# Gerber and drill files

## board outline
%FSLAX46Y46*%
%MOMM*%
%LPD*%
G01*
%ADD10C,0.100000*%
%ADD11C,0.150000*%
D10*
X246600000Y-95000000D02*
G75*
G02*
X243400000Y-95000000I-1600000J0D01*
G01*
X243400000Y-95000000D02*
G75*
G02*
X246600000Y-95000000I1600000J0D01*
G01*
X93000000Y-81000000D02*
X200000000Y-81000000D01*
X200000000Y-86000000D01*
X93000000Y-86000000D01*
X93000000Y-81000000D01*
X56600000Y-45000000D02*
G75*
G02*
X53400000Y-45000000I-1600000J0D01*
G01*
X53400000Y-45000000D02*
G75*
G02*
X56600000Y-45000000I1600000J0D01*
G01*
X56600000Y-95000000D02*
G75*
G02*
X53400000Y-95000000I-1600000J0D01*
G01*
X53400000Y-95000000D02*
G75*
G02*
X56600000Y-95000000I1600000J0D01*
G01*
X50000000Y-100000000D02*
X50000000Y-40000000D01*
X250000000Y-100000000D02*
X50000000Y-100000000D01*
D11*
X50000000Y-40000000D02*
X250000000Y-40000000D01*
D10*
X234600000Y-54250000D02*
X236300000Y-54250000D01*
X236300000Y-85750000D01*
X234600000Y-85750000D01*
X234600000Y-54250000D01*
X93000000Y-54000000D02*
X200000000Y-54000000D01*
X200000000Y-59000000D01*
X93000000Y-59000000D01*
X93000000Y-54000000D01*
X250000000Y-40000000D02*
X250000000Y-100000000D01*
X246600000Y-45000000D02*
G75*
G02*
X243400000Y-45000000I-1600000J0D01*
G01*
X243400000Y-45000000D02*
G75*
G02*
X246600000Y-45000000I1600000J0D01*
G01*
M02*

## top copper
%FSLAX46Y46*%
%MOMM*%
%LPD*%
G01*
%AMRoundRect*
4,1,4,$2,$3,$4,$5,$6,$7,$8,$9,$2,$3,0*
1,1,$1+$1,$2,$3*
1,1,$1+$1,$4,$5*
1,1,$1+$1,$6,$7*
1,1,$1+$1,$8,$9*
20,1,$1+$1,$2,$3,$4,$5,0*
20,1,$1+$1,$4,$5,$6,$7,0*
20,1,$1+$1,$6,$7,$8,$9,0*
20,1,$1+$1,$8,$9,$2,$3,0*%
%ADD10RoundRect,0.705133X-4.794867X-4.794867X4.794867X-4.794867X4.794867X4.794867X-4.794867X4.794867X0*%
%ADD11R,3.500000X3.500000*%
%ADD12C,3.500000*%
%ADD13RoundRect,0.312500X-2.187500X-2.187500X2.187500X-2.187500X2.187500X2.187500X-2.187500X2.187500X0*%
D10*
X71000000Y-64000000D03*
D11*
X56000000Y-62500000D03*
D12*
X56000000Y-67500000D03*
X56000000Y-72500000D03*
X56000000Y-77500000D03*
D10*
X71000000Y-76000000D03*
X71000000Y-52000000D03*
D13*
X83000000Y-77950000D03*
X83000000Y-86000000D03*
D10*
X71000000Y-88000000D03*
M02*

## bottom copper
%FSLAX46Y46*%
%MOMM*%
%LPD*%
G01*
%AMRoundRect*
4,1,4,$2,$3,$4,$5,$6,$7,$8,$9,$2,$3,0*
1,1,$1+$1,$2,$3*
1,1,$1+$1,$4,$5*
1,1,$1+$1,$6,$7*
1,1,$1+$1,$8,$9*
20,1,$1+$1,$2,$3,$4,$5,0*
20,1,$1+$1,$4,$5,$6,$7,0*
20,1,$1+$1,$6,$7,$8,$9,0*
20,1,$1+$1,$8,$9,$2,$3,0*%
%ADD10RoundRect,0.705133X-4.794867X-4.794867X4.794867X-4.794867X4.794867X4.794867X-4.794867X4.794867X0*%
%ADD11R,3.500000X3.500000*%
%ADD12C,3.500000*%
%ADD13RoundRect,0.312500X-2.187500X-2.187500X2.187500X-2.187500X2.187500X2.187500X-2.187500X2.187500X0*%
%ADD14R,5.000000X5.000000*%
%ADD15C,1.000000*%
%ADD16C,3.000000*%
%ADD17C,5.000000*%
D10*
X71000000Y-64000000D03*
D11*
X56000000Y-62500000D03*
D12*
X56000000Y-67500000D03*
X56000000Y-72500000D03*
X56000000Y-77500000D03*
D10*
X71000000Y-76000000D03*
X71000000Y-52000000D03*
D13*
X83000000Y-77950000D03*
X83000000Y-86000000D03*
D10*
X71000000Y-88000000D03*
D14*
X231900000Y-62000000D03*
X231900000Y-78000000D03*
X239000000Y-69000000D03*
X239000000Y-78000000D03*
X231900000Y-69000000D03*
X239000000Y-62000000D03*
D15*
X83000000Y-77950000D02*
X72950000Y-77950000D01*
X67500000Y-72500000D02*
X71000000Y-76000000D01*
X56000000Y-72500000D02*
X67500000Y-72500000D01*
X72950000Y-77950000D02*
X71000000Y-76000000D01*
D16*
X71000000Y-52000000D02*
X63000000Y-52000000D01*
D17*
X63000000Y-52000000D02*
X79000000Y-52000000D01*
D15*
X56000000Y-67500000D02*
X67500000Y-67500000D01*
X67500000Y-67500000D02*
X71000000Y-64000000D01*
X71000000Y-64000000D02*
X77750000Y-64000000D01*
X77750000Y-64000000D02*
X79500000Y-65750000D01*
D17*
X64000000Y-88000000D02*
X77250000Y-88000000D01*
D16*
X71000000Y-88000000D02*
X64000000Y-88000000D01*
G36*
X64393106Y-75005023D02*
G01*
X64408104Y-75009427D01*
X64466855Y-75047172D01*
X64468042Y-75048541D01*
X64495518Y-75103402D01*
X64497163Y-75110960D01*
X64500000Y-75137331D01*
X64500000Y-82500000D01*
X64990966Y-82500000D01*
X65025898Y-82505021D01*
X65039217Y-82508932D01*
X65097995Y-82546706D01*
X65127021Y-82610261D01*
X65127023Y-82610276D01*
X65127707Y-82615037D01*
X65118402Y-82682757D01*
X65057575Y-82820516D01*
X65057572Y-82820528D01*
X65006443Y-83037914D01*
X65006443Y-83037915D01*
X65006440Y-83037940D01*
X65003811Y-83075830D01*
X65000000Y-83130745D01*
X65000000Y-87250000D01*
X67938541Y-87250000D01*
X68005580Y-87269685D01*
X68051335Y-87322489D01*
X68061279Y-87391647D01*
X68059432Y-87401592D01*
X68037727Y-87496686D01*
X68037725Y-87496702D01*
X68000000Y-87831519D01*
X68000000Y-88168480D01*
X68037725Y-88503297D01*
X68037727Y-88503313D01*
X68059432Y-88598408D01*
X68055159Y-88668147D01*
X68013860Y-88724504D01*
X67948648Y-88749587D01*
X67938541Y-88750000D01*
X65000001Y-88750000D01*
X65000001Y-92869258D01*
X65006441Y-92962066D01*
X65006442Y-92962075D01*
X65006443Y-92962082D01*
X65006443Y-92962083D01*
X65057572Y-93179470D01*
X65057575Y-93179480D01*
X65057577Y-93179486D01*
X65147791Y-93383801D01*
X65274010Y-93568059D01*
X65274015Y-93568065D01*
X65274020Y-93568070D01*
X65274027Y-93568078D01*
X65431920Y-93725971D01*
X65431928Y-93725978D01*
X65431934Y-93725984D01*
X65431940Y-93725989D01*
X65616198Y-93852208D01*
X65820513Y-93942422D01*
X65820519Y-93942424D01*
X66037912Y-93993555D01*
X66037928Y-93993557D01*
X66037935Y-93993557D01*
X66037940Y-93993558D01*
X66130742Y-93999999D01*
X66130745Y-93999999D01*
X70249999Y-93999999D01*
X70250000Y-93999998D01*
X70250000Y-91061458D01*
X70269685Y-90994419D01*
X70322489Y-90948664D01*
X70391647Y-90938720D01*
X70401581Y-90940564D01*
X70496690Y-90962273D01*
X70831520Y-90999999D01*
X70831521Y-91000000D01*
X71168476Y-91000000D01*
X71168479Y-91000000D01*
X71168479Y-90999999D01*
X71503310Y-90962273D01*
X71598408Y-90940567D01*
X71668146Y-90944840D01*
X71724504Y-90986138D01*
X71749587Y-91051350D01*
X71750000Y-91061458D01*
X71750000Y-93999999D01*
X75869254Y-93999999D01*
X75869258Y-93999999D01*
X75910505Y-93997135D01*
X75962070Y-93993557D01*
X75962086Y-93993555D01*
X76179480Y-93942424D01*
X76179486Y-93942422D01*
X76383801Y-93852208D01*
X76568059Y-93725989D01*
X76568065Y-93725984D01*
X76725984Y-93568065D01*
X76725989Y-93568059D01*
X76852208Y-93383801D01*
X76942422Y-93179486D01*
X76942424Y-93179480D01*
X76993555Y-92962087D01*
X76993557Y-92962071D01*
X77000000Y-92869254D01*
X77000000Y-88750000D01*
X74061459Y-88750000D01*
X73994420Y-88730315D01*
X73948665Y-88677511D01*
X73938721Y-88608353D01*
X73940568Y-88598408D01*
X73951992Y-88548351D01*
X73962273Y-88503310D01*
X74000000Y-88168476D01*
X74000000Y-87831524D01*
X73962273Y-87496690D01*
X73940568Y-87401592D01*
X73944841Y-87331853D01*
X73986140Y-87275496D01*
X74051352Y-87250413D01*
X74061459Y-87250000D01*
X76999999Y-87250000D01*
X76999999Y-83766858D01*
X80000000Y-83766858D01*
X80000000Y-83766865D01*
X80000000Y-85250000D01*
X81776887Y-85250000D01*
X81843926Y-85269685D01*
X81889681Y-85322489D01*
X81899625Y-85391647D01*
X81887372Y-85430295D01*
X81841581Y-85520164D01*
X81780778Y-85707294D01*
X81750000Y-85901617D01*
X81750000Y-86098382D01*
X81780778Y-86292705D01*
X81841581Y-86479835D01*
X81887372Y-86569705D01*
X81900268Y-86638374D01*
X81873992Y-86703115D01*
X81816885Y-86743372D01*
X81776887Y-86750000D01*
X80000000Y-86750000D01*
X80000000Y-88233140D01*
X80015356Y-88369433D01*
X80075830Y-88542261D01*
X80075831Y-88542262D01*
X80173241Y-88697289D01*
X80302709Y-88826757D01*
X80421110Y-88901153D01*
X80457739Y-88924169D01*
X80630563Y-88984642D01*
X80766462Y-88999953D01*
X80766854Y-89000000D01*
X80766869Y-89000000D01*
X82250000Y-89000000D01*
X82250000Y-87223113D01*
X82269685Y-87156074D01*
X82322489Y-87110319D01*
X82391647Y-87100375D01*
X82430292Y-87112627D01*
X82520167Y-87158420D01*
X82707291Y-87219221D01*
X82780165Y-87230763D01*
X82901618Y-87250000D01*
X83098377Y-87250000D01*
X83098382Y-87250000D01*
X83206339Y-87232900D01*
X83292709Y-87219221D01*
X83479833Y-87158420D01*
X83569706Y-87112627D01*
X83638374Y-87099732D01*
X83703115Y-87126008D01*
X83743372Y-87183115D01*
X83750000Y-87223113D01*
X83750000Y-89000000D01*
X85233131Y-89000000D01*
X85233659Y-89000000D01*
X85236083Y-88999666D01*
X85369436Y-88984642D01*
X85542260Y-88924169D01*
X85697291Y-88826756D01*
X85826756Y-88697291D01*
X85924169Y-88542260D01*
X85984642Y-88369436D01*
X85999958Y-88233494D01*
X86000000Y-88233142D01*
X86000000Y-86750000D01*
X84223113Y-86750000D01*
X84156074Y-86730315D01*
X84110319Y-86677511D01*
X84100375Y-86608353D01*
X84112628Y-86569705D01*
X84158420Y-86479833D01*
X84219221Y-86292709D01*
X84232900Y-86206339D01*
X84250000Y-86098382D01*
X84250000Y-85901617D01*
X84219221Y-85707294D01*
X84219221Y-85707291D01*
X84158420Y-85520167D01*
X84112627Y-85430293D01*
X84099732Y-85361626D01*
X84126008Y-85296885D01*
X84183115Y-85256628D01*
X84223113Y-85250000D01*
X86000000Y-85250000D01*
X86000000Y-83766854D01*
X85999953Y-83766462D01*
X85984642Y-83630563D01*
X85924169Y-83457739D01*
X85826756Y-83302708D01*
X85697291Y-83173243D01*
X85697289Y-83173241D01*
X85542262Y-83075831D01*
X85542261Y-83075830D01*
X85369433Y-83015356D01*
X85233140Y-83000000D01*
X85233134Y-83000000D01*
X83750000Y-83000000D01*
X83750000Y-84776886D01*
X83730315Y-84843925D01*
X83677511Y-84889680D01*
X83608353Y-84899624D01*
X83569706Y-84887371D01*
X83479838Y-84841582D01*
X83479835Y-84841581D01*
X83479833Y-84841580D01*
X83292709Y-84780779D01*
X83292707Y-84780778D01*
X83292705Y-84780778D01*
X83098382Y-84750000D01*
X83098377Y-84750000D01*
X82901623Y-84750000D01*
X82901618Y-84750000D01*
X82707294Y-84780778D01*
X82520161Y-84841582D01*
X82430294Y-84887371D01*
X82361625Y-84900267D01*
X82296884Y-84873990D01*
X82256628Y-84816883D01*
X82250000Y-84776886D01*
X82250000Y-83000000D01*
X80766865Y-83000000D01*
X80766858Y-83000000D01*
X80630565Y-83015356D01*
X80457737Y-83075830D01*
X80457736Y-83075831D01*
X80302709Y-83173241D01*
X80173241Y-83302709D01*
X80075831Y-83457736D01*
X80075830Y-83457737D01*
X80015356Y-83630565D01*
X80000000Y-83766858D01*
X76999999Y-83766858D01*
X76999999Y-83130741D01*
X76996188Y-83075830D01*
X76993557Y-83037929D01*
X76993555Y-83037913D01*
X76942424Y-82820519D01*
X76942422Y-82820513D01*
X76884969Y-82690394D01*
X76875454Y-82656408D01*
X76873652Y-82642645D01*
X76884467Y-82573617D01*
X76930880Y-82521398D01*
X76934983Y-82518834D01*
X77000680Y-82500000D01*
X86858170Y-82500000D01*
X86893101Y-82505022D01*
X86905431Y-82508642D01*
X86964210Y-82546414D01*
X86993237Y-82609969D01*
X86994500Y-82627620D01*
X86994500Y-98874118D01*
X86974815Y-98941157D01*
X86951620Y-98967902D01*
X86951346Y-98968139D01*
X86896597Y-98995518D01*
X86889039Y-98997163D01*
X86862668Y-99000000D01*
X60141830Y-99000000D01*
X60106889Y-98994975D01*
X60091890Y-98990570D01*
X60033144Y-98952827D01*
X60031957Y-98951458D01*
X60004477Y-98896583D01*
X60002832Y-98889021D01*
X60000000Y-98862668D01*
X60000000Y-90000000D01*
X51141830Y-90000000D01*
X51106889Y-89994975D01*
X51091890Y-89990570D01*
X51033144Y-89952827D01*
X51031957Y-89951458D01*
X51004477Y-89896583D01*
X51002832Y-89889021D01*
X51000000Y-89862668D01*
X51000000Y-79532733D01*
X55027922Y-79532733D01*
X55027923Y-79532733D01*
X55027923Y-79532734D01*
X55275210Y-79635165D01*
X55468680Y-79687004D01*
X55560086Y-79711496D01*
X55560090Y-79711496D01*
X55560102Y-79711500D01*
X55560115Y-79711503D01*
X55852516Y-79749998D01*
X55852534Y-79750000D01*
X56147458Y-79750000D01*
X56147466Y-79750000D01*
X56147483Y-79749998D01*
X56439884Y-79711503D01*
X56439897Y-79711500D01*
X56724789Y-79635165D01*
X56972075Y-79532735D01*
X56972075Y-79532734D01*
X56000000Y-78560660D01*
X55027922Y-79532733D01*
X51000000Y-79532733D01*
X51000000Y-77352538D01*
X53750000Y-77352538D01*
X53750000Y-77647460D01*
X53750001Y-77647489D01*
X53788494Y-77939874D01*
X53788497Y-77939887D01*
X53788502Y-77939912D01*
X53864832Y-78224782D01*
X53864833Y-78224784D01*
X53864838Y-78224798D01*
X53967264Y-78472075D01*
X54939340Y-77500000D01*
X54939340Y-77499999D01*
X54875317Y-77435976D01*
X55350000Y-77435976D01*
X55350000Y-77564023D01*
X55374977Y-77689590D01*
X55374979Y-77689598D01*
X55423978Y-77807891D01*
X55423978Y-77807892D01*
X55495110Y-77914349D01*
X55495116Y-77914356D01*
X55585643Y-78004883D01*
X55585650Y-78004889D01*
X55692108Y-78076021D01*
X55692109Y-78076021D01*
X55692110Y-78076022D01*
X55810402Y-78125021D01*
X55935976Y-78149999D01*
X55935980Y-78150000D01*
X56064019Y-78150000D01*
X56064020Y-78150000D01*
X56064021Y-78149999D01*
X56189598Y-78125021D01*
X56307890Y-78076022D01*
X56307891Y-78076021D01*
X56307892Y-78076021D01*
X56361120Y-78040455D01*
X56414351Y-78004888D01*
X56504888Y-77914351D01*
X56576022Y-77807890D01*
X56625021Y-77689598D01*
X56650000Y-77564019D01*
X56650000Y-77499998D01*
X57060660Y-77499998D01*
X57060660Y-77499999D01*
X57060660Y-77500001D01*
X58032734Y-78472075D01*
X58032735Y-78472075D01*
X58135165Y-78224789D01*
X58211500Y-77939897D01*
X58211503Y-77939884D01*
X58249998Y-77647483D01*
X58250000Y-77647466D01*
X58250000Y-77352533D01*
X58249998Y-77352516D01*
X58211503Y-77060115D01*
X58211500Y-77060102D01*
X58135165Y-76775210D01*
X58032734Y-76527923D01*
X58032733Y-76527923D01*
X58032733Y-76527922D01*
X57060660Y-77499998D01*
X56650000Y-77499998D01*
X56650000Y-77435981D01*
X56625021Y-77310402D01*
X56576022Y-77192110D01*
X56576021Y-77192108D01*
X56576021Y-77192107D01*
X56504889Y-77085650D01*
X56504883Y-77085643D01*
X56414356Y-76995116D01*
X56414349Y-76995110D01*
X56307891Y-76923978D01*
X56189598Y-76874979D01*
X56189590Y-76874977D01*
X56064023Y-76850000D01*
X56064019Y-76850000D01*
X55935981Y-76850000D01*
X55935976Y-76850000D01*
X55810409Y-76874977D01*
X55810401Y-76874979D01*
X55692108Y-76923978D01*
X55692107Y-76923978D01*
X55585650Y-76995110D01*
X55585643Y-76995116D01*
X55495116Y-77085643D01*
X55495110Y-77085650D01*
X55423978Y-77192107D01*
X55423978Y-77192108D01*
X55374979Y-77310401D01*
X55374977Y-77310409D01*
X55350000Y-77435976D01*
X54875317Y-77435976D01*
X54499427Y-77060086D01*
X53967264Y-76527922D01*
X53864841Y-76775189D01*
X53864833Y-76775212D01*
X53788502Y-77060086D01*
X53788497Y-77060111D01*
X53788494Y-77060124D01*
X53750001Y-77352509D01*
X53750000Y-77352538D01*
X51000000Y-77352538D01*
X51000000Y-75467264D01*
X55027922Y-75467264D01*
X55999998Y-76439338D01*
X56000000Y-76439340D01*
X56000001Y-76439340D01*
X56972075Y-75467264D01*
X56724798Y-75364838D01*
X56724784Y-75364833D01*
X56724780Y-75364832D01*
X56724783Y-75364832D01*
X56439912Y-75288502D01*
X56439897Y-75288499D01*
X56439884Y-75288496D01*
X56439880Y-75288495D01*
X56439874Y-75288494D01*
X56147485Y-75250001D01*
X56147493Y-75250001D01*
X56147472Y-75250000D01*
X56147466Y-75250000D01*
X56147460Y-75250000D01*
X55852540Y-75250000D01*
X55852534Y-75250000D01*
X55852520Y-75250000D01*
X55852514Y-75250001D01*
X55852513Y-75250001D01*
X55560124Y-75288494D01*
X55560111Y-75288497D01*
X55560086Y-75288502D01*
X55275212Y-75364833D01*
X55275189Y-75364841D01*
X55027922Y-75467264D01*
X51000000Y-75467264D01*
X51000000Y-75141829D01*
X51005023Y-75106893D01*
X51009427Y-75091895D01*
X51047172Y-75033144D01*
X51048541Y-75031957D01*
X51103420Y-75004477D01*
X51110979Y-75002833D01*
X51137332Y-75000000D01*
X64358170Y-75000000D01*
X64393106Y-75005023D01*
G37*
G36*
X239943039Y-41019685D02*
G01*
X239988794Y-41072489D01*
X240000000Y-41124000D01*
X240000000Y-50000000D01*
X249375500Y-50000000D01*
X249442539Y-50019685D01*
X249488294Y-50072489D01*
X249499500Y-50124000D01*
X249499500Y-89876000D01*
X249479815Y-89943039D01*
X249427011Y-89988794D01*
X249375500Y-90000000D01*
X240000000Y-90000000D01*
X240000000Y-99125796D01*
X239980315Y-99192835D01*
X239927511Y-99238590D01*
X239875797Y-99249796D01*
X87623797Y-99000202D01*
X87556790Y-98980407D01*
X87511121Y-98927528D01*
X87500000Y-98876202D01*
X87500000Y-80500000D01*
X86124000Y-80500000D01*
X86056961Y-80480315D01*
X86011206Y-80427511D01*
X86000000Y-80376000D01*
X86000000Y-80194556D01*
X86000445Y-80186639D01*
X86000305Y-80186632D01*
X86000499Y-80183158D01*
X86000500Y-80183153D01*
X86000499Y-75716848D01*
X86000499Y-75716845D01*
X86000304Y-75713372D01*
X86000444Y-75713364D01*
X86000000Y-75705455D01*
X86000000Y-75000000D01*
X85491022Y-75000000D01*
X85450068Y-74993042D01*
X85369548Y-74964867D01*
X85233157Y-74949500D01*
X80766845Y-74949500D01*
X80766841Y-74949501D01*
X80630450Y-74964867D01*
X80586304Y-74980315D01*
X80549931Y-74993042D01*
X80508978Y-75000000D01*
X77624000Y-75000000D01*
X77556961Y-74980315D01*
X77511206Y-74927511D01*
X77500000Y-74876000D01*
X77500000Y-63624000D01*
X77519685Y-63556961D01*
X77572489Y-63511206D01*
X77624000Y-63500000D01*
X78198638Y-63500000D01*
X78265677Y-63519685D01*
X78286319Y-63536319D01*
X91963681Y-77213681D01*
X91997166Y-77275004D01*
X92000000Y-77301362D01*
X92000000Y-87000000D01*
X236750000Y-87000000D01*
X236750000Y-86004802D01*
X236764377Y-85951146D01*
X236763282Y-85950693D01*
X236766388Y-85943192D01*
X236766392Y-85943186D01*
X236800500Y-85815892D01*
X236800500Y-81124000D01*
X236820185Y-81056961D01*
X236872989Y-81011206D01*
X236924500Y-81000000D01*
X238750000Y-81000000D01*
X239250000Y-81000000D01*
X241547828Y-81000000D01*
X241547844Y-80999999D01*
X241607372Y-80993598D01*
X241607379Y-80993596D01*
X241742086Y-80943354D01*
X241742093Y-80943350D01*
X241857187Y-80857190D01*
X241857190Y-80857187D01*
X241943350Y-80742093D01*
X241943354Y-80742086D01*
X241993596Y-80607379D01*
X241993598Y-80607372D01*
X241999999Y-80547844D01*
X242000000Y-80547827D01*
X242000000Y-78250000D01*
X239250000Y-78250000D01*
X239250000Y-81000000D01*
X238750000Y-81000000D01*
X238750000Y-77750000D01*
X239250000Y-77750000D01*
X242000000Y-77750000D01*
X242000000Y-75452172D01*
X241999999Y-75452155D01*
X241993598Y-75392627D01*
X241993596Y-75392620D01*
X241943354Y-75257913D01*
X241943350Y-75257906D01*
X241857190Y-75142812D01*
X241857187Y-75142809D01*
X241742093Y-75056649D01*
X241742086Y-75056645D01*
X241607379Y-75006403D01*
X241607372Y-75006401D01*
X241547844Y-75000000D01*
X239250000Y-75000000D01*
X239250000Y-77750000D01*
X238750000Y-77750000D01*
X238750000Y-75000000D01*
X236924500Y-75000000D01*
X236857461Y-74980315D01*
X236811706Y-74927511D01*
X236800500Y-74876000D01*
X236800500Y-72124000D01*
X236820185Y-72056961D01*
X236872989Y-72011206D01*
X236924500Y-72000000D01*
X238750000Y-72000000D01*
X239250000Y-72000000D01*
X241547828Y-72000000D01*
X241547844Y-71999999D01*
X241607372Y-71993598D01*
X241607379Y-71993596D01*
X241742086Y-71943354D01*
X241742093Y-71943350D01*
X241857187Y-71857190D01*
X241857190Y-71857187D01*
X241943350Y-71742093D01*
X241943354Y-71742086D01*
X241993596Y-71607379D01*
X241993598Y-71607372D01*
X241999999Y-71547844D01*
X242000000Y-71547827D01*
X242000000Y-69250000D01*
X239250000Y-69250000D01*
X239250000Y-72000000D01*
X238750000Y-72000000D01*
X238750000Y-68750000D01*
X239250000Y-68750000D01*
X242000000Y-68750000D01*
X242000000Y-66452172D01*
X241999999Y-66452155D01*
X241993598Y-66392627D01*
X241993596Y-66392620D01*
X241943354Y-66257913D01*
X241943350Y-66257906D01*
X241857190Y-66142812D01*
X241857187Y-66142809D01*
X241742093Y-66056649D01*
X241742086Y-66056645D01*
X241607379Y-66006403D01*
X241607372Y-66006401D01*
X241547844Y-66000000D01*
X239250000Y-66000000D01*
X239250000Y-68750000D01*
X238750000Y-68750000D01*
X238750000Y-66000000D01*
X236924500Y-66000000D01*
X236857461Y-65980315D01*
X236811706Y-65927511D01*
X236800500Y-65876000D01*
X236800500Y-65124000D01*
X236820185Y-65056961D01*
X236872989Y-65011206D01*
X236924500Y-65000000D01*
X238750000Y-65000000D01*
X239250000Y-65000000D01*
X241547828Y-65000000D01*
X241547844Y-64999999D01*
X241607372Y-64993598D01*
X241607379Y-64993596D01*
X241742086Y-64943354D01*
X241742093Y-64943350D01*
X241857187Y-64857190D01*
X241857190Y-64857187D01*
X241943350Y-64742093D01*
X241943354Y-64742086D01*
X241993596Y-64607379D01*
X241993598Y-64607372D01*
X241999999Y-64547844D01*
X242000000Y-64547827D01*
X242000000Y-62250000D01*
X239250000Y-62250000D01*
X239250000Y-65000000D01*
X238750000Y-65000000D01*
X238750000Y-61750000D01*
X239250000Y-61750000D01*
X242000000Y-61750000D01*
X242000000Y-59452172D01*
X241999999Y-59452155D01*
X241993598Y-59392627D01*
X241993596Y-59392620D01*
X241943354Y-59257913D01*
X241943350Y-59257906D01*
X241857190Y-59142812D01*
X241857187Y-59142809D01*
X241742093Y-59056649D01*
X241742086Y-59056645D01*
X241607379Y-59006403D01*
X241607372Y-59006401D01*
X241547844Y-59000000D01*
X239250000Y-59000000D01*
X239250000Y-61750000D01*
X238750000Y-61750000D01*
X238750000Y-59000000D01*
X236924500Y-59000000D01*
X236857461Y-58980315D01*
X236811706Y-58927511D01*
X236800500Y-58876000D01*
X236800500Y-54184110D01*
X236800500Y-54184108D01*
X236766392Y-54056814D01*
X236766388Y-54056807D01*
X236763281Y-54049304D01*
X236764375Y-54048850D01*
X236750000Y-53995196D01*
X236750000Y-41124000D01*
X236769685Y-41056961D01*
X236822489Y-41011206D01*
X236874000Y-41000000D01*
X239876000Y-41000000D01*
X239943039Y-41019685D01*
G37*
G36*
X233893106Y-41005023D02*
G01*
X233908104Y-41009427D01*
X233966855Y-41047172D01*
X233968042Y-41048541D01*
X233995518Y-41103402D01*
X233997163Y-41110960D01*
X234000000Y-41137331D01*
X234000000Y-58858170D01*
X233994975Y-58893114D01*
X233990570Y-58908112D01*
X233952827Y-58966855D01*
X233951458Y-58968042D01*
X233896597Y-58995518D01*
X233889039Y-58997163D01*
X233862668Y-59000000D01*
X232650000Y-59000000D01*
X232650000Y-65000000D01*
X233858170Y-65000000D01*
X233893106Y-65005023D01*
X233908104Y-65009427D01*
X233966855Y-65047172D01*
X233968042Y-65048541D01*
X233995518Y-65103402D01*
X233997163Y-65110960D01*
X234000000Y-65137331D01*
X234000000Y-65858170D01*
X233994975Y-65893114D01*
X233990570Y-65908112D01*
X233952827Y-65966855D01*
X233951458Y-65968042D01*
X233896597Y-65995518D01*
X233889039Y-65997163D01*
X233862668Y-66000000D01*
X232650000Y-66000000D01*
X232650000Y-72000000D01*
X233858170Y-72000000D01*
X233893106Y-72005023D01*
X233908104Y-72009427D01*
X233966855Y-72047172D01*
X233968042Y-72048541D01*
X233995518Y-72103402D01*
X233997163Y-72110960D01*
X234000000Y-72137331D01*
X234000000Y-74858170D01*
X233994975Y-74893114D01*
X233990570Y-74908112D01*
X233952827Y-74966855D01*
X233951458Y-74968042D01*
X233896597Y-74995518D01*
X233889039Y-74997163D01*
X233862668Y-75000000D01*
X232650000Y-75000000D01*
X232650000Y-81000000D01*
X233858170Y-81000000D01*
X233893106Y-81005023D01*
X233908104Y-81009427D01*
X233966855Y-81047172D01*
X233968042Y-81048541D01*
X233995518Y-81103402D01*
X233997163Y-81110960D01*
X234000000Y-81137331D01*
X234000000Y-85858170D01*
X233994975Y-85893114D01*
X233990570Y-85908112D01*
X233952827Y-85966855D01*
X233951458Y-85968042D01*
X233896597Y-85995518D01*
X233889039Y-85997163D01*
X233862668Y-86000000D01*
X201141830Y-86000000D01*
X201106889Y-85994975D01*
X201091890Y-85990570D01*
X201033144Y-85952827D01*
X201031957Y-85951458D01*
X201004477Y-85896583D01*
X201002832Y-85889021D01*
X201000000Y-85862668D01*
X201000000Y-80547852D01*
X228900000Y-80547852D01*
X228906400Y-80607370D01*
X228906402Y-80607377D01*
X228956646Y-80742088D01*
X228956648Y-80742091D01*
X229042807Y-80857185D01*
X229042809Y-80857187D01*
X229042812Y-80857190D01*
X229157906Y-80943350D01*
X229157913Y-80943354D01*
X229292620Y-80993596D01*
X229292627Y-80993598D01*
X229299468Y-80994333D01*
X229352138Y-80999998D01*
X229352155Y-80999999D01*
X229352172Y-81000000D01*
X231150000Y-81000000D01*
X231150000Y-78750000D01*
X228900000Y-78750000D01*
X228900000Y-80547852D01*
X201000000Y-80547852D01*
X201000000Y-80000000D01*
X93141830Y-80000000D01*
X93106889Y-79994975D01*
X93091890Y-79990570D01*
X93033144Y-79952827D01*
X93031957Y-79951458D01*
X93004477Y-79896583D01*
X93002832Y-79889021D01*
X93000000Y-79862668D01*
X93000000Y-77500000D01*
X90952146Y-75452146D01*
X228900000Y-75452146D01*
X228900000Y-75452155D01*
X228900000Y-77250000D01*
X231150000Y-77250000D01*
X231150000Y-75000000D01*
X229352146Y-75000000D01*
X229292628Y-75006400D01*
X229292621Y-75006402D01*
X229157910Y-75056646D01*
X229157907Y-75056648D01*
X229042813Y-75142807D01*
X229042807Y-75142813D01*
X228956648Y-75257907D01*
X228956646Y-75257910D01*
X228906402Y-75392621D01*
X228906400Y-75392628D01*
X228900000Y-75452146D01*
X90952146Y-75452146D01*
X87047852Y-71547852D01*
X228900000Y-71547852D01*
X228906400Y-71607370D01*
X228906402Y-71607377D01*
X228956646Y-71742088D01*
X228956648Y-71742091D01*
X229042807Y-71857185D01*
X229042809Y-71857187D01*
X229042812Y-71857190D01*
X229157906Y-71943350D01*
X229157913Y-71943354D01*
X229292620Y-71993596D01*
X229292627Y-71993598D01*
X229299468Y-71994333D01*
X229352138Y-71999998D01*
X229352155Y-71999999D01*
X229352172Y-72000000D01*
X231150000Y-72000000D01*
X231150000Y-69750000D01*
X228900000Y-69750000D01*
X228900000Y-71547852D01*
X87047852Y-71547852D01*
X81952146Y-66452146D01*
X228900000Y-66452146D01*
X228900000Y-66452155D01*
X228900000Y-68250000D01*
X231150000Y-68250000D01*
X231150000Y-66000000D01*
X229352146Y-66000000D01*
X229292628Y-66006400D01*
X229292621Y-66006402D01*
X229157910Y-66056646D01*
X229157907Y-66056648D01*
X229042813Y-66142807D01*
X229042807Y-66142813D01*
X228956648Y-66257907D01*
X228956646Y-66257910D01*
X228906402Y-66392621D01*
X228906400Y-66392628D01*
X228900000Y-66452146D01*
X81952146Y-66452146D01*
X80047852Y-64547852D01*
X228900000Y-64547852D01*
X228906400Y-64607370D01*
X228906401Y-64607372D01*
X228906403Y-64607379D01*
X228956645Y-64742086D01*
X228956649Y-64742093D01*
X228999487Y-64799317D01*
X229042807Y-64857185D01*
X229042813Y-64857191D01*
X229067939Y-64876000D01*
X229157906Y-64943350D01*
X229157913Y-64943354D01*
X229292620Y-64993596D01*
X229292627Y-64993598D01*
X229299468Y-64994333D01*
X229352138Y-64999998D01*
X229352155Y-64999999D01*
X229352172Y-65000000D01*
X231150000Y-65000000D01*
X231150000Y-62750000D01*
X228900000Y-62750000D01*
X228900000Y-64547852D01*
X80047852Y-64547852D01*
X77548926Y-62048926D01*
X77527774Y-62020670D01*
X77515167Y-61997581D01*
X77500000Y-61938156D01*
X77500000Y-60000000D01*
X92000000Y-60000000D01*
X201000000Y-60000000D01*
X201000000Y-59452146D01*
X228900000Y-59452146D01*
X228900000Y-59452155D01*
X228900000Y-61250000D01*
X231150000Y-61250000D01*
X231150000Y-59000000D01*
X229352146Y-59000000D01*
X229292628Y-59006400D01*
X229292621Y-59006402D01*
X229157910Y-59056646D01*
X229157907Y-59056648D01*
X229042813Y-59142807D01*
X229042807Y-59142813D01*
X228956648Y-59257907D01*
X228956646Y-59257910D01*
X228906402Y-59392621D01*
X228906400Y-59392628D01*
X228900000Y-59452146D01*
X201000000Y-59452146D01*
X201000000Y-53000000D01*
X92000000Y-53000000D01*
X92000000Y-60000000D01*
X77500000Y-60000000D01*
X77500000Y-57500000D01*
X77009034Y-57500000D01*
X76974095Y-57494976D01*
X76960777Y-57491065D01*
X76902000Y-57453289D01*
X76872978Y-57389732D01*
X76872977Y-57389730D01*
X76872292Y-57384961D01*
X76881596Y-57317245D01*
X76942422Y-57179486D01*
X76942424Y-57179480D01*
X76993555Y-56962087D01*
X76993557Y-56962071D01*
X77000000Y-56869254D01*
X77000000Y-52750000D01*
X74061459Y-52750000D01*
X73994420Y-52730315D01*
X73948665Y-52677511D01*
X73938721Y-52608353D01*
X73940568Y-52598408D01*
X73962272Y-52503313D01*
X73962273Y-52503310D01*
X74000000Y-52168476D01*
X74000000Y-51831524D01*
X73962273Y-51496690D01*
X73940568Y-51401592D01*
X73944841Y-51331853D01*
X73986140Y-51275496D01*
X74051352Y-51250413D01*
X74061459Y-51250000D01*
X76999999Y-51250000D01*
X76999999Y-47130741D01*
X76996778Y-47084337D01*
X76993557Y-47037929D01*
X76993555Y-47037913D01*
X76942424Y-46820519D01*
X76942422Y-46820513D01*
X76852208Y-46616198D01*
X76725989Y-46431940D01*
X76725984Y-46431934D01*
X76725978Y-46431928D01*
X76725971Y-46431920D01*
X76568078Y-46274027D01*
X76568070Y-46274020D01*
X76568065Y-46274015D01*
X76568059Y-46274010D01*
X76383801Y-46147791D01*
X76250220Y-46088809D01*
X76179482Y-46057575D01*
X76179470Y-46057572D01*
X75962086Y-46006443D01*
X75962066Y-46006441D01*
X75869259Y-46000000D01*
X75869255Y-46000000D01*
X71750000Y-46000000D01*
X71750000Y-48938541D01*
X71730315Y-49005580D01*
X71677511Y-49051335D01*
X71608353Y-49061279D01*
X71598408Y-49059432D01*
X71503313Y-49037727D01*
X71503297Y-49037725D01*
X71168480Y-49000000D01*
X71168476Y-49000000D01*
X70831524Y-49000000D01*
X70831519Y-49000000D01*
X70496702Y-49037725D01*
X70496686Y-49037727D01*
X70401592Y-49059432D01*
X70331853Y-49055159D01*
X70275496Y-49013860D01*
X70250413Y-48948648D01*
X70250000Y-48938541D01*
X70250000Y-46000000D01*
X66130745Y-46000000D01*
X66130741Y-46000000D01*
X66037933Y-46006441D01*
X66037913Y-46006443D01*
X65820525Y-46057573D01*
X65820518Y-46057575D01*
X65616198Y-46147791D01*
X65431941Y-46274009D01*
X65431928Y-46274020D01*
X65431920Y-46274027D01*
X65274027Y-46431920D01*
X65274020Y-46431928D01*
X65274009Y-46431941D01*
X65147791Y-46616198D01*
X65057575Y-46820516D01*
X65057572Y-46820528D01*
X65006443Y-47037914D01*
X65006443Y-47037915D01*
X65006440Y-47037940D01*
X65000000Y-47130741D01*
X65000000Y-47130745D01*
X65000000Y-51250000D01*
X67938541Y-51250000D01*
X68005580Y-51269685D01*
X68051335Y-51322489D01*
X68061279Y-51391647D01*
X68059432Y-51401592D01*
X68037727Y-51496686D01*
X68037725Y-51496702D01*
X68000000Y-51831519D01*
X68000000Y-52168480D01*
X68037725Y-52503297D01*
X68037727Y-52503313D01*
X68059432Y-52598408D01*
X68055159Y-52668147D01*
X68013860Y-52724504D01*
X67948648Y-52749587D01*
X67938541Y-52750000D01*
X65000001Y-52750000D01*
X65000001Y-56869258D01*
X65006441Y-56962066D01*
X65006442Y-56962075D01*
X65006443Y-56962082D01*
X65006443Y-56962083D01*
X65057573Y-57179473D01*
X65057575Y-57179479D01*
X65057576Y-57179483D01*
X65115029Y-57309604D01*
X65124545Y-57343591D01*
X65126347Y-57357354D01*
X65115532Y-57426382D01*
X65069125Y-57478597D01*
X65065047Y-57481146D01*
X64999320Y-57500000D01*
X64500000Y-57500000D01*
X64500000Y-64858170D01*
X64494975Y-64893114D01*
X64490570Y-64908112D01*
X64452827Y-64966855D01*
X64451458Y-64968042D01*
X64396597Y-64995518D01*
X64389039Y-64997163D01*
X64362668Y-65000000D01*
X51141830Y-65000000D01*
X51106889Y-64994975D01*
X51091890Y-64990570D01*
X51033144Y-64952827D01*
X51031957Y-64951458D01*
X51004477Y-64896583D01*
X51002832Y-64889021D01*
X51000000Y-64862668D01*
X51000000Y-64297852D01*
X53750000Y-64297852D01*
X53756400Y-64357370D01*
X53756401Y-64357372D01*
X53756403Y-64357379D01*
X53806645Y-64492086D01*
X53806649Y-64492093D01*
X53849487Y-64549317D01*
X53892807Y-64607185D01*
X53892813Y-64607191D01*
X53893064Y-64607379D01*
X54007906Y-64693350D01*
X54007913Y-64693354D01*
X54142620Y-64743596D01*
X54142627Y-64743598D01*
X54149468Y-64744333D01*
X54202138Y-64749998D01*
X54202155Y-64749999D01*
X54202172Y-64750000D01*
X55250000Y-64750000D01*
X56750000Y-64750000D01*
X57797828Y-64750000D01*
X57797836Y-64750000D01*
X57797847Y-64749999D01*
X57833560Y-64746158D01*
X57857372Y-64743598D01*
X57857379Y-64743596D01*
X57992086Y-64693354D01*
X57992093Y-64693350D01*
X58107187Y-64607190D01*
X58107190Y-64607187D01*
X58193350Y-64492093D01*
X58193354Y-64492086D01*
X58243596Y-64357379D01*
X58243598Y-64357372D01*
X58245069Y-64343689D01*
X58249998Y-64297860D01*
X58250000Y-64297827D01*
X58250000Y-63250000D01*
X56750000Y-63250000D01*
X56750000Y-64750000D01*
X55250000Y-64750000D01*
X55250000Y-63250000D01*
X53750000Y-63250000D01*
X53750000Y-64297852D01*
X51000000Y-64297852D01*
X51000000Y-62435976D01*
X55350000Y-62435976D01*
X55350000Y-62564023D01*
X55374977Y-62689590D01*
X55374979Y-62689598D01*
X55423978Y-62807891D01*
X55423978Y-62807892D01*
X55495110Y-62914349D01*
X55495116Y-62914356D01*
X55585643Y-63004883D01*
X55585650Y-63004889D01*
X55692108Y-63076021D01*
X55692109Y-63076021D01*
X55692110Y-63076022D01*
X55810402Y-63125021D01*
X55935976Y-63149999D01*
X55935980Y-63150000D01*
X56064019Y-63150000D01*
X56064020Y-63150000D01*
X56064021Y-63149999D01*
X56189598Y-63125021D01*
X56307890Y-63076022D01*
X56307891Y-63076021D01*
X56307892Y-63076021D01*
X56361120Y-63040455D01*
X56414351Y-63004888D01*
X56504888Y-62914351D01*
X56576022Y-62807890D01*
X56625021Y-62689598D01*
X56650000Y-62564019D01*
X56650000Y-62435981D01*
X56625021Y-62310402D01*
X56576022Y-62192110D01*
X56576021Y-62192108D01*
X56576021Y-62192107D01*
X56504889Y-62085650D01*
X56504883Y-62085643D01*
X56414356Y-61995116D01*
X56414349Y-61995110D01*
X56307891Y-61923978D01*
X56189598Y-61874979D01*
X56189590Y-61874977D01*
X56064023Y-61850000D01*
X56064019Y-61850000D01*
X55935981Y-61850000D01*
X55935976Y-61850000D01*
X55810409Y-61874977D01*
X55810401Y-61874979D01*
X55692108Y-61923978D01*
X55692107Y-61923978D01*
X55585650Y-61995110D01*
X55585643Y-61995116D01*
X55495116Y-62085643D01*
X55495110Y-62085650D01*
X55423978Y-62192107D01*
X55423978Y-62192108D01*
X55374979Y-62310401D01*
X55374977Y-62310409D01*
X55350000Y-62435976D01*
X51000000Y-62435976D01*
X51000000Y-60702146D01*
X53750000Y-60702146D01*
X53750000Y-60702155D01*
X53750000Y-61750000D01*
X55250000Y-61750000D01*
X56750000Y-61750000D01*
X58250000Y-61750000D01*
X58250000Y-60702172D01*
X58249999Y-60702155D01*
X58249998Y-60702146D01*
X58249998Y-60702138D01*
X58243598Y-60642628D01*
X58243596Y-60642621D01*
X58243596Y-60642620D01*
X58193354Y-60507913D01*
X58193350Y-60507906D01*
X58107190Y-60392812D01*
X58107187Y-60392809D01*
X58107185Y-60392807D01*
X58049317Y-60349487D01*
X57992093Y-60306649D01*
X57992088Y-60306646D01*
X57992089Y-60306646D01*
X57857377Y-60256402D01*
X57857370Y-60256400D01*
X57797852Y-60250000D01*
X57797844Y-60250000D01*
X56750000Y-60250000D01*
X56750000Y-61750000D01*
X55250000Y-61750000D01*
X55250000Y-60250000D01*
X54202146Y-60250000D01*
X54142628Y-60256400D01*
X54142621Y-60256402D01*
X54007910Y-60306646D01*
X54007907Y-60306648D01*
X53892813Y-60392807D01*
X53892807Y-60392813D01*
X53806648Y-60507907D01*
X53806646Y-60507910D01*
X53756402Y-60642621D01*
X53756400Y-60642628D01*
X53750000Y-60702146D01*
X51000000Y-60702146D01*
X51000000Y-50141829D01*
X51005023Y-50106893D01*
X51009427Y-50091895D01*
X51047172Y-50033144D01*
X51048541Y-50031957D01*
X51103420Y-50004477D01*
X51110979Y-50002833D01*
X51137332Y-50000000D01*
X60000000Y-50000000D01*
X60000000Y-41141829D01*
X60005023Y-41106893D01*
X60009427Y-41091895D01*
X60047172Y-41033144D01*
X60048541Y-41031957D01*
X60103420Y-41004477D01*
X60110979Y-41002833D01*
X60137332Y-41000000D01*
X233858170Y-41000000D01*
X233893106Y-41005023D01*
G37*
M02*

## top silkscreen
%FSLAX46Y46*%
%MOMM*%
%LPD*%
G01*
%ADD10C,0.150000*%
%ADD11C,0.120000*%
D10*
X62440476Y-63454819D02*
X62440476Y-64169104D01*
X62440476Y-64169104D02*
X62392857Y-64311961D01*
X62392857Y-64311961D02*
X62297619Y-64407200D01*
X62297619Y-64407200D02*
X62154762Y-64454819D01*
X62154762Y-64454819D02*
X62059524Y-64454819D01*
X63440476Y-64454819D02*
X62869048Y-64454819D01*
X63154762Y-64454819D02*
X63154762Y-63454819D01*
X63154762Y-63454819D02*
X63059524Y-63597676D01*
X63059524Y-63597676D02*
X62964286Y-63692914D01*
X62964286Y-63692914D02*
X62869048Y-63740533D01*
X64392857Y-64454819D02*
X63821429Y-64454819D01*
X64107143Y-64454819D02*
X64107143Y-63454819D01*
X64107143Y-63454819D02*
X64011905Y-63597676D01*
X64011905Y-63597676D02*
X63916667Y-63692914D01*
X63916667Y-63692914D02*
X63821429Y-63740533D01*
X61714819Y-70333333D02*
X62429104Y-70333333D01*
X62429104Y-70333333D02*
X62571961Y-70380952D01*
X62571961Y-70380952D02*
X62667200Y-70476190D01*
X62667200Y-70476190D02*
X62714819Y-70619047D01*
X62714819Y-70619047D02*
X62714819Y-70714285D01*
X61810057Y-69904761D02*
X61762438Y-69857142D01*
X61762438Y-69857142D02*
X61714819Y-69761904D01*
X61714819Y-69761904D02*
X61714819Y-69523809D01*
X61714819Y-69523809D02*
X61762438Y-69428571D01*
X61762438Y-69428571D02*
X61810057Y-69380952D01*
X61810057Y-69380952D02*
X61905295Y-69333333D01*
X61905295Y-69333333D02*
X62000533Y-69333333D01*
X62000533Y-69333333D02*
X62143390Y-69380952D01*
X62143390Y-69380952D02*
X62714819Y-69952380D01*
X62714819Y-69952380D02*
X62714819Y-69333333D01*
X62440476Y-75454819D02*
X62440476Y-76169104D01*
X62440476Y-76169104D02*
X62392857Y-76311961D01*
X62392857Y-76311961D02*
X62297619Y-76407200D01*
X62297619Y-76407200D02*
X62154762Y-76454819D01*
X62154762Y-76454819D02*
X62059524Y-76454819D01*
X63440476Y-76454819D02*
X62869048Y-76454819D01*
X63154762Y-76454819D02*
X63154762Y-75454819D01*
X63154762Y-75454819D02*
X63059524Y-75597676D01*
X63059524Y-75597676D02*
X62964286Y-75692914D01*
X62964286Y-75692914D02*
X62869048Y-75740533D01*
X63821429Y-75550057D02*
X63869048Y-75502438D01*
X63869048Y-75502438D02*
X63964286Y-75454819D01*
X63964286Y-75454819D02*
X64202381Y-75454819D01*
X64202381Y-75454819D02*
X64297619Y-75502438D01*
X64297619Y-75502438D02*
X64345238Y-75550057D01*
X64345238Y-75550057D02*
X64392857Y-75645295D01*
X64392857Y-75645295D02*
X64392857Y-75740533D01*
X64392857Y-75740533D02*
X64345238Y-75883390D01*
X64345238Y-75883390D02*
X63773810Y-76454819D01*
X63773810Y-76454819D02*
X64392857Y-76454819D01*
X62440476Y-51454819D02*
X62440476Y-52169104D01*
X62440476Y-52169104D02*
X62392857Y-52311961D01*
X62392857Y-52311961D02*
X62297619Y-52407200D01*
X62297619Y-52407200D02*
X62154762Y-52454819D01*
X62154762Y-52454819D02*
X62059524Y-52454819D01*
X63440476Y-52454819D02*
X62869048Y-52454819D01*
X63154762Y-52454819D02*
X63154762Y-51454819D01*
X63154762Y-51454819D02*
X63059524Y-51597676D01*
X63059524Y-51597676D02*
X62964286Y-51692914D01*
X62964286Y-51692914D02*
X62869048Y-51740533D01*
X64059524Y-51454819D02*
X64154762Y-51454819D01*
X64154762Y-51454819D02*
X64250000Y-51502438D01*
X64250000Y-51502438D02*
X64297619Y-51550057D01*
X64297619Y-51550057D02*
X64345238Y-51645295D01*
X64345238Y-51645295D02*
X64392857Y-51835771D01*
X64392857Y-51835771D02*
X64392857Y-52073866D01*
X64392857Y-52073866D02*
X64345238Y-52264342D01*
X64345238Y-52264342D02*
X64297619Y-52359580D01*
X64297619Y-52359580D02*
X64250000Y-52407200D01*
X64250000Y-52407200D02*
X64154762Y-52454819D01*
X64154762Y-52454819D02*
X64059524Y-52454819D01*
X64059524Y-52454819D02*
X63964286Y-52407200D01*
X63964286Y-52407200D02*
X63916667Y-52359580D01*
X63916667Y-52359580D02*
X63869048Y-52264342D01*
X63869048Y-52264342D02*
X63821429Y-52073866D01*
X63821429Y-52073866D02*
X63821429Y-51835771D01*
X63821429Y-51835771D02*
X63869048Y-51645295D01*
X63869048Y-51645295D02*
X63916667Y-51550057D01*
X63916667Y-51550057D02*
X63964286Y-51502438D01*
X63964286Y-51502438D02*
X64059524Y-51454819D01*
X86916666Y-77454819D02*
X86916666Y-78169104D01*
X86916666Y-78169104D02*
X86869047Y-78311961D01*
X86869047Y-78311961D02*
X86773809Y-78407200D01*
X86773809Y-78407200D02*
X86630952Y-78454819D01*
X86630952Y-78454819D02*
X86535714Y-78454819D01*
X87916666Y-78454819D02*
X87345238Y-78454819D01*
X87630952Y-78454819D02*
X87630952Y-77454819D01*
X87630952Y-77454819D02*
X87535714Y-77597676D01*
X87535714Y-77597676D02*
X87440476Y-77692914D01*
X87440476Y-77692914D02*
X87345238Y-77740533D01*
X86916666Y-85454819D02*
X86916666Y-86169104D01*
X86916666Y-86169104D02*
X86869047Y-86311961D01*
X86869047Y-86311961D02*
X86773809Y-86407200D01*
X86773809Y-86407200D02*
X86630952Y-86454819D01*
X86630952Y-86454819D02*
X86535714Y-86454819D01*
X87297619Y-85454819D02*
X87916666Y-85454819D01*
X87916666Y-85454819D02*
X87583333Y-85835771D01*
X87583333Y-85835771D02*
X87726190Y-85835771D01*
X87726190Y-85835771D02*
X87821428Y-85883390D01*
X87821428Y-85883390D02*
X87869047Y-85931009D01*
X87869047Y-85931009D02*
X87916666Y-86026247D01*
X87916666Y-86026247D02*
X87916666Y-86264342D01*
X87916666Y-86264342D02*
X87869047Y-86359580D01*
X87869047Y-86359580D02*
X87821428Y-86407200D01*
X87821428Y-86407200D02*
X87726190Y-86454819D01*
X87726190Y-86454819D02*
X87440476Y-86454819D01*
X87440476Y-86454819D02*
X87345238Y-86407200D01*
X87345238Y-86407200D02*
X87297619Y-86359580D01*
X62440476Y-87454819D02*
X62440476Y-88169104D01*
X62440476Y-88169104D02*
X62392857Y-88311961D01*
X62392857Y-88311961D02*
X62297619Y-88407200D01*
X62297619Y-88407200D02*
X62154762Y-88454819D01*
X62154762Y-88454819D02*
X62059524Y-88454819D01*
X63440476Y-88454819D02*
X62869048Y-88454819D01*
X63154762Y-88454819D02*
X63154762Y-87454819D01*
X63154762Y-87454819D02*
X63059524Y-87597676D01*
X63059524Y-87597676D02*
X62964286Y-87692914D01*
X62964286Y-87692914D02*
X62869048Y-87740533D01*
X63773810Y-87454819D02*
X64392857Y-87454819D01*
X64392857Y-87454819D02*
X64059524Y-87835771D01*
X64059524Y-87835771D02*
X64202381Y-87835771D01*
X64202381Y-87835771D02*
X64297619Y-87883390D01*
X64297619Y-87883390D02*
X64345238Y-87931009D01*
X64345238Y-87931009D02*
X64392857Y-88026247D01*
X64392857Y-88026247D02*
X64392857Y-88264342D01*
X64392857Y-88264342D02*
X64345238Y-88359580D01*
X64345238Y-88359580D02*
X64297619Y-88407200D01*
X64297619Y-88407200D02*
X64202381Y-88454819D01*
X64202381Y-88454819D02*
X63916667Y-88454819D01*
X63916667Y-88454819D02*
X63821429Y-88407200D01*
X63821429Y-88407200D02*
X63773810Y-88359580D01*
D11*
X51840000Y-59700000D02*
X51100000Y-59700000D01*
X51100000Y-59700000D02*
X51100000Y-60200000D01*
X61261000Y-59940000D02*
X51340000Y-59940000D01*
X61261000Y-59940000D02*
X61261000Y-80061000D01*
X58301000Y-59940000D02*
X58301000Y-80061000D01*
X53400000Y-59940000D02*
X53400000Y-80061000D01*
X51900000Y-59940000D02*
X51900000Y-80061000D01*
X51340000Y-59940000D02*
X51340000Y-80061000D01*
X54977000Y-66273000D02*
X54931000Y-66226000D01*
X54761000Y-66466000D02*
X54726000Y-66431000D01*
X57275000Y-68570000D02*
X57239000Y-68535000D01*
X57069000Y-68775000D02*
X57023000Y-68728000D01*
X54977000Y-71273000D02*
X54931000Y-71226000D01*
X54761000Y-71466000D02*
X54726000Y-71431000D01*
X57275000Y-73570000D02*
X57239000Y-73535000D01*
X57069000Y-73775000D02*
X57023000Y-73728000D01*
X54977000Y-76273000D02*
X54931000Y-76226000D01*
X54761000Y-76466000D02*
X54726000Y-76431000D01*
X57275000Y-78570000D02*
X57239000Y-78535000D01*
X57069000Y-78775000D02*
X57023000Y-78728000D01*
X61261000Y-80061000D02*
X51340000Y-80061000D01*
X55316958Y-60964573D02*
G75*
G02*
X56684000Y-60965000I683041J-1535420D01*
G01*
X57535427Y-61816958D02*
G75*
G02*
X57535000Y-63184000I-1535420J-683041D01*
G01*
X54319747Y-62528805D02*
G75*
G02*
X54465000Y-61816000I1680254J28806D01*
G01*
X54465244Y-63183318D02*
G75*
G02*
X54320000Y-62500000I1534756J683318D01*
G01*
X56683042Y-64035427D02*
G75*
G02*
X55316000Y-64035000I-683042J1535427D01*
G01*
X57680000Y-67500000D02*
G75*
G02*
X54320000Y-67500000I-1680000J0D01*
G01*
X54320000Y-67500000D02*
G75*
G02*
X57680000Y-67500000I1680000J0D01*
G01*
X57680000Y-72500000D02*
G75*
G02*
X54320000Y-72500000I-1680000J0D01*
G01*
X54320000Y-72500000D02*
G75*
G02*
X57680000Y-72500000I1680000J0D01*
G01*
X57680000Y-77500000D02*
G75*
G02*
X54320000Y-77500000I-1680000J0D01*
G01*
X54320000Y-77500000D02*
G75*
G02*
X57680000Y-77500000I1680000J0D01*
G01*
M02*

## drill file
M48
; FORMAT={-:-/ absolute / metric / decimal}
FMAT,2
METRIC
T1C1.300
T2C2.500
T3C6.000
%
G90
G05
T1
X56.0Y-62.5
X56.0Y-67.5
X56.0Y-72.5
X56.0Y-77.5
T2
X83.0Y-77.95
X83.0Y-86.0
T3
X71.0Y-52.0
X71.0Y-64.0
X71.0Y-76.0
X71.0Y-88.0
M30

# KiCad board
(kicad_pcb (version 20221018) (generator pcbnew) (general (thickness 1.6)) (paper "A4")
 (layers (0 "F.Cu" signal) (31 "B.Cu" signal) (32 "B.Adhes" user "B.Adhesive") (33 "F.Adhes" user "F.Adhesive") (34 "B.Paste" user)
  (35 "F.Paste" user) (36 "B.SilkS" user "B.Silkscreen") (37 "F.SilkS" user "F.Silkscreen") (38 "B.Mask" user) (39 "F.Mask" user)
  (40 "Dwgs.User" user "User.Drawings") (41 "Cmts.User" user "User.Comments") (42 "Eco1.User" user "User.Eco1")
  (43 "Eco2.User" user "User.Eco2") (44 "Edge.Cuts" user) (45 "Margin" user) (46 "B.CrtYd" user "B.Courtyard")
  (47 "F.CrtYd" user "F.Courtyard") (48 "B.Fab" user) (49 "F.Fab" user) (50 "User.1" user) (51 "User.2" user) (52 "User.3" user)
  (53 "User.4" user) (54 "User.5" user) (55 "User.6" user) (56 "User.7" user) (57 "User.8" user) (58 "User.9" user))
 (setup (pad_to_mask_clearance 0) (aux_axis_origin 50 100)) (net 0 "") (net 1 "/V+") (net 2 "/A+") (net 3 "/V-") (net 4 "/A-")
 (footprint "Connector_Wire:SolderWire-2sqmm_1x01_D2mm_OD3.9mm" (layer "F.Cu") (at 71 64)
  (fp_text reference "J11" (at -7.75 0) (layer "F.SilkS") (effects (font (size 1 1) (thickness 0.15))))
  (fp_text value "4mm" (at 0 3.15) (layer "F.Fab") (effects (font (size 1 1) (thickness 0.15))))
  (pad "1" thru_hole roundrect (at 0 0) (size 11 11) (drill 6) (layers "*.Cu" "*.Mask") (roundrect_rratio 0.064103) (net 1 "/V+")))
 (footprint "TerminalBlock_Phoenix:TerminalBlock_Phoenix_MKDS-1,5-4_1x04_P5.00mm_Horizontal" (layer "F.Cu") (at 56 62.5 -90)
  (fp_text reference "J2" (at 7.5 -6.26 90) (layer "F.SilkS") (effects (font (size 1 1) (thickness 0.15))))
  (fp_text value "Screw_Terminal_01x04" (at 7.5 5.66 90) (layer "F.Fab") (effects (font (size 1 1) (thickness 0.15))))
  (fp_line (start -2.8 4.16) (end -2.8 4.9) (stroke (width 0.12) (type solid)) (layer "F.SilkS"))
  (fp_line (start -2.8 4.9) (end -2.3 4.9) (stroke (width 0.12) (type solid)) (layer "F.SilkS"))
  (fp_line (start -2.56 -5.261) (end -2.56 4.66) (stroke (width 0.12) (type solid)) (layer "F.SilkS"))
  (fp_line (start -2.56 -5.261) (end 17.561 -5.261) (stroke (width 0.12) (type solid)) (layer "F.SilkS"))
  (fp_line (start -2.56 -2.301) (end 17.561 -2.301) (stroke (width 0.12) (type solid)) (layer "F.SilkS"))
  (fp_line (start -2.56 2.6) (end 17.561 2.6) (stroke (width 0.12) (type solid)) (layer "F.SilkS"))
  (fp_line (start -2.56 4.1) (end 17.561 4.1) (stroke (width 0.12) (type solid)) (layer "F.SilkS"))
  (fp_line (start -2.56 4.66) (end 17.561 4.66) (stroke (width 0.12) (type solid)) (layer "F.SilkS"))
  (fp_line (start 3.773 1.023) (end 3.726 1.069) (stroke (width 0.12) (type solid)) (layer "F.SilkS"))
  (fp_line (start 3.966 1.239) (end 3.931 1.274) (stroke (width 0.12) (type solid)) (layer "F.SilkS"))
  (fp_line (start 6.07 -1.275) (end 6.035 -1.239) (stroke (width 0.12) (type solid)) (layer "F.SilkS"))
  (fp_line (start 6.275 -1.069) (end 6.228 -1.023) (stroke (width 0.12) (type solid)) (layer "F.SilkS"))
  (fp_line (start 8.773 1.023) (end 8.726 1.069) (stroke (width 0.12) (type solid)) (layer "F.SilkS"))
  (fp_line (start 8.966 1.239) (end 8.931 1.274) (stroke (width 0.12) (type solid)) (layer "F.SilkS"))
  (fp_line (start 11.07 -1.275) (end 11.035 -1.239) (stroke (width 0.12) (type solid)) (layer "F.SilkS"))
  (fp_line (start 11.275 -1.069) (end 11.228 -1.023) (stroke (width 0.12) (type solid)) (layer "F.SilkS"))
  (fp_line (start 13.773 1.023) (end 13.726 1.069) (stroke (width 0.12) (type solid)) (layer "F.SilkS"))
  (fp_line (start 13.966 1.239) (end 13.931 1.274) (stroke (width 0.12) (type solid)) (layer "F.SilkS"))
  (fp_line (start 16.07 -1.275) (end 16.035 -1.239) (stroke (width 0.12) (type solid)) (layer "F.SilkS"))
  (fp_line (start 16.275 -1.069) (end 16.228 -1.023) (stroke (width 0.12) (type solid)) (layer "F.SilkS"))
  (fp_line (start 17.561 -5.261) (end 17.561 4.66) (stroke (width 0.12) (type solid)) (layer "F.SilkS"))
  (fp_arc (start -1.535427 0.683042) (mid -1.680501 -0.000524) (end -1.535 -0.684) (stroke (width 0.12) (type solid)) (layer "F.SilkS"))
  (fp_arc (start -0.683042 -1.535427) (mid 0.000524 -1.680501) (end 0.684 -1.535) (stroke (width 0.12) (type solid)) (layer "F.SilkS"))
  (fp_arc (start 0.028805 1.680253) (mid -0.335551 1.646659) (end -0.684 1.535) (stroke (width 0.12) (type solid)) (layer "F.SilkS"))
  (fp_arc (start 0.683318 1.534756) (mid 0.349292 1.643288) (end 0 1.68) (stroke (width 0.12) (type solid)) (layer "F.SilkS"))
  (fp_arc (start 1.535427 -0.683042) (mid 1.680501 0.000524) (end 1.535 0.684) (stroke (width 0.12) (type solid)) (layer "F.SilkS"))
  (fp_circle (center 5 0) (end 6.68 0) (stroke (width 0.12) (type solid)) (fill none) (layer "F.SilkS"))
  (fp_circle (center 10 0) (end 11.68 0) (stroke (width 0.12) (type solid)) (fill none) (layer "F.SilkS"))
  (fp_circle (center 15 0) (end 16.68 0) (stroke (width 0.12) (type solid)) (fill none) (layer "F.SilkS"))
  (pad "1" thru_hole rect (at 0 0 270) (size 3.5 3.5) (drill 1.3) (layers "*.Cu" "*.Mask") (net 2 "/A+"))
  (pad "2" thru_hole circle (at 5 0 270) (size 3.5 3.5) (drill 1.3) (layers "*.Cu" "*.Mask") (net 1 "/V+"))
  (pad "3" thru_hole circle (at 10 0 270) (size 3.5 3.5) (drill 1.3) (layers "*.Cu" "*.Mask") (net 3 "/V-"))
  (pad "4" thru_hole circle (at 15 0 270) (size 3.5 3.5) (drill 1.3) (layers "*.Cu" "*.Mask") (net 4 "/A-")))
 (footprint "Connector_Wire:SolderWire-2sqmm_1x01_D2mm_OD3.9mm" (layer "F.Cu") (at 71 76)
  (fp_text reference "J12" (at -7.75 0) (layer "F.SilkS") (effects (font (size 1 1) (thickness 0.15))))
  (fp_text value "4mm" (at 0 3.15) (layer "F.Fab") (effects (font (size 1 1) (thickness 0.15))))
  (pad "1" thru_hole roundrect (at 0 0) (size 11 11) (drill 6) (layers "*.Cu" "*.Mask") (roundrect_rratio 0.064103) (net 3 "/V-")))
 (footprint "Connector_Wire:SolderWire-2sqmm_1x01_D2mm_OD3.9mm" (layer "F.Cu") (at 71 52)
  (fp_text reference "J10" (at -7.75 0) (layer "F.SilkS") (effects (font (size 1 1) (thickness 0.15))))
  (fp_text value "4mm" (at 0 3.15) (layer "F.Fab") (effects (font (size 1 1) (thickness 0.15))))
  (pad "1" thru_hole roundrect (at 0 0) (size 11 11) (drill 6) (layers "*.Cu" "*.Mask") (roundrect_rratio 0.064103) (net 2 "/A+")))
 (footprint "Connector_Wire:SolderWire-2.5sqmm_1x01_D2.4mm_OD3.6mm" (layer "F.Cu") (at 83 77.95)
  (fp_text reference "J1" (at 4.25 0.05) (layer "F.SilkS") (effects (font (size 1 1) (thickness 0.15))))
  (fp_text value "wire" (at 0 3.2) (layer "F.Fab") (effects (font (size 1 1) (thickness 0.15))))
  (pad "1" thru_hole roundrect (at 0 0) (size 5 5) (drill 2.5) (layers "*.Cu" "*.Mask") (roundrect_rratio 0.0625) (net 3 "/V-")))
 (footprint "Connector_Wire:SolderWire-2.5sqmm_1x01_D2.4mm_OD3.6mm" (layer "F.Cu") (at 83 86)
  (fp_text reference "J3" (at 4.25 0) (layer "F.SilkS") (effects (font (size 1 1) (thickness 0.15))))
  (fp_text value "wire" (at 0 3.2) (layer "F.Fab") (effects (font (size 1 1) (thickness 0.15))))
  (pad "1" thru_hole roundrect (at 0 0) (size 5 5) (drill 2.5) (layers "*.Cu" "*.Mask") (roundrect_rratio 0.0625) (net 4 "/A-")))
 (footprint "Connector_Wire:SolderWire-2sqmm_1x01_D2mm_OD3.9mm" (layer "F.Cu") (at 71 88)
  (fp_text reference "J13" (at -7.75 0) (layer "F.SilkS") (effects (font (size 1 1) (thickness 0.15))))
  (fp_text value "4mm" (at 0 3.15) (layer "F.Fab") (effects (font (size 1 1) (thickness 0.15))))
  (pad "1" thru_hole roundrect (at 0 0) (size 11 11) (drill 6) (layers "*.Cu" "*.Mask") (roundrect_rratio 0.064103) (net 4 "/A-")))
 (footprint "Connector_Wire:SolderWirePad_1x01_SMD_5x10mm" (layer "B.Cu") (at 231.9 62 180)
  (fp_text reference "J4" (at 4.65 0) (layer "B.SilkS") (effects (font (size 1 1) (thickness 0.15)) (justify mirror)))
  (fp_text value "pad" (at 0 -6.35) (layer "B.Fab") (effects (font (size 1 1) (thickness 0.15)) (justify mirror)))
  (pad "1" smd rect (at 0 0 180) (size 5 5) (layers "B.Cu" "B.Paste" "B.Mask") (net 2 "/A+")))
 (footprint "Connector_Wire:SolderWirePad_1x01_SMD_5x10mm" (layer "B.Cu") (at 231.9 78 180)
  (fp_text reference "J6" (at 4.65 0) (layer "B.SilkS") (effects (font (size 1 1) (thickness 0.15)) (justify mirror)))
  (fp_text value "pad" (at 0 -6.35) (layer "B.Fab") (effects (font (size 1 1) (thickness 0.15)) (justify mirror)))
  (pad "1" smd rect (at 0 0 180) (size 5 5) (layers "B.Cu" "B.Paste" "B.Mask") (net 2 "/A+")))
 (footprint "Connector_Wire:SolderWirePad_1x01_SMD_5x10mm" (layer "B.Cu") (at 239 69 180)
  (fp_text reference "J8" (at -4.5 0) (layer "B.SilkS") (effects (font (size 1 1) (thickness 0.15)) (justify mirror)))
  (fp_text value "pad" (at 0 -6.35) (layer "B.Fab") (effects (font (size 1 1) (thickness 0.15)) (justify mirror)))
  (pad "1" smd rect (at 0 0 180) (size 5 5) (layers "B.Cu" "B.Paste" "B.Mask") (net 1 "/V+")))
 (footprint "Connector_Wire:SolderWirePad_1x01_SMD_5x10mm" (layer "B.Cu") (at 239 78 180)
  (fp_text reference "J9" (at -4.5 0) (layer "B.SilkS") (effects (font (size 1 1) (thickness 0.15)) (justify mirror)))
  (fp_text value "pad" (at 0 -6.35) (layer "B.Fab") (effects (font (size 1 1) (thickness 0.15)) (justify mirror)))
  (pad "1" smd rect (at 0 0 180) (size 5 5) (layers "B.Cu" "B.Paste" "B.Mask") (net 1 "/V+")))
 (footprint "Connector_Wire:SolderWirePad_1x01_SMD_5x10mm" (layer "B.Cu") (at 231.9 69 180)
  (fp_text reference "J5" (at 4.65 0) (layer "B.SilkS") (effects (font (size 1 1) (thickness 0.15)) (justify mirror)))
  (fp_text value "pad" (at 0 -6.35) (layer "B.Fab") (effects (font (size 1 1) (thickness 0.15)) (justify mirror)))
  (pad "1" smd rect (at 0 0 180) (size 5 5) (layers "B.Cu" "B.Paste" "B.Mask") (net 2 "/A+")))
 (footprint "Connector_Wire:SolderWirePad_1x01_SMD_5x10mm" (layer "B.Cu") (at 239 62 180)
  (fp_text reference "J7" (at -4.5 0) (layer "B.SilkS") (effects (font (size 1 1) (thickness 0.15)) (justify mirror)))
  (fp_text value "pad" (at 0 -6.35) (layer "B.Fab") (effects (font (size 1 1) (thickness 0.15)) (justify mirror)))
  (pad "1" smd rect (at 0 0 180) (size 5 5) (layers "B.Cu" "B.Paste" "B.Mask") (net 1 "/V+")))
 (gr_circle (center 245 95) (end 246.6 95) (stroke (width 0.1) (type default)) (fill none) (layer "Edge.Cuts"))
 (gr_rect (start 93 81) (end 200 86) (stroke (width 0.1) (type default)) (fill none) (layer "Edge.Cuts"))
 (gr_circle (center 55 45) (end 56.6 45) (stroke (width 0.1) (type default)) (fill none) (layer "Edge.Cuts"))
 (gr_circle (center 55 95) (end 56.6 95) (stroke (width 0.1) (type default)) (fill none) (layer "Edge.Cuts"))
 (gr_line (start 50 100) (end 50 40) (stroke (width 0.1) (type default)) (layer "Edge.Cuts"))
 (gr_line (start 250 100) (end 50 100) (stroke (width 0.1) (type default)) (layer "Edge.Cuts"))
 (gr_line (start 50 40) (end 250 40) (stroke (width 0.15) (type default)) (layer "Edge.Cuts"))
 (gr_rect (start 234.6 54.25) (end 236.3 85.75) (stroke (width 0.1) (type default)) (fill none) (layer "Edge.Cuts"))
 (gr_rect (start 93 54) (end 200 59) (stroke (width 0.1) (type default)) (fill none) (layer "Edge.Cuts"))
 (gr_line (start 250 40) (end 250 100) (stroke (width 0.1) (type default)) (layer "Edge.Cuts"))
 (gr_circle (center 245 45) (end 246.6 45) (stroke (width 0.1) (type default)) (fill none) (layer "Edge.Cuts"))
 (segment (start 83 77.95) (end 72.95 77.95) (width 1) (layer "B.Cu") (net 3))
 (segment (start 67.5 72.5) (end 71 76) (width 1) (layer "B.Cu") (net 3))
 (segment (start 56 72.5) (end 67.5 72.5) (width 1) (layer "B.Cu") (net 3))
 (segment (start 72.95 77.95) (end 71 76) (width 1) (layer "B.Cu") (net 3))
 (segment (start 71 52) (end 63 52) (width 3) (layer "B.Cu") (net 2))
 (segment (start 63 52) (end 79 52) (width 5) (layer "B.Cu") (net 2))
 (segment (start 56 67.5) (end 67.5 67.5) (width 1) (layer "B.Cu") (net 1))
 (segment (start 67.5 67.5) (end 71 64) (width 1) (layer "B.Cu") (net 1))
 (segment (start 71 64) (end 77.75 64) (width 1) (layer "B.Cu") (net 1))
 (segment (start 77.75 64) (end 79.5 65.75) (width 1) (layer "B.Cu") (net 1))
 (segment (start 64 88) (end 77.25 88) (width 5) (layer "B.Cu") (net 4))
 (segment (start 71 88) (end 64 88) (width 3) (layer "B.Cu") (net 4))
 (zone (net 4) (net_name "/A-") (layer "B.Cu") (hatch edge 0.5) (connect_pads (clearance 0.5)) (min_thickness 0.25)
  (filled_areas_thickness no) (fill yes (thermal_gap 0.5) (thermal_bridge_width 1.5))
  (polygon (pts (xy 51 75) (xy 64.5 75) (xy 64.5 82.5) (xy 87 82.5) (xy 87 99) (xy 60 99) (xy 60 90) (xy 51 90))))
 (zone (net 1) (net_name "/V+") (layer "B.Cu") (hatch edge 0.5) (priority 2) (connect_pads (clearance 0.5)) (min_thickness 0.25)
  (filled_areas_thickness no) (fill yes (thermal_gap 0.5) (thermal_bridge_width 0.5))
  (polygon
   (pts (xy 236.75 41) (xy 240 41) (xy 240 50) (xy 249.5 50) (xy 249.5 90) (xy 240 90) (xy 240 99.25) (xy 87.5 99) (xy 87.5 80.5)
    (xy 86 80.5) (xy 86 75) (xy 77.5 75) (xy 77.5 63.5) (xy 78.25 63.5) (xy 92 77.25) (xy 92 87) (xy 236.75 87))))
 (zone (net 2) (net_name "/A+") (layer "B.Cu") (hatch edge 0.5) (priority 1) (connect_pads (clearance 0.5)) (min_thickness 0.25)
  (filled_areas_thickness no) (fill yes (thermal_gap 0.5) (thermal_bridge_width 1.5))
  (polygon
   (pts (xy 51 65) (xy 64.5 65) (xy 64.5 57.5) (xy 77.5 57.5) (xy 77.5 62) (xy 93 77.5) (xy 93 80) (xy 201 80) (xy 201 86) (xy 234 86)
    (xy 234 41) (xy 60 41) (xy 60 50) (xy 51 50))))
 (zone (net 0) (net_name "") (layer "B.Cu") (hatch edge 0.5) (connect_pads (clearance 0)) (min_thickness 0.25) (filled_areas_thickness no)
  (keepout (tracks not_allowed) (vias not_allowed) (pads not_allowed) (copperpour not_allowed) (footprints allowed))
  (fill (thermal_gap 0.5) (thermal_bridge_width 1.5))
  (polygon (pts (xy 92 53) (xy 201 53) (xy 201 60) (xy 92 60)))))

